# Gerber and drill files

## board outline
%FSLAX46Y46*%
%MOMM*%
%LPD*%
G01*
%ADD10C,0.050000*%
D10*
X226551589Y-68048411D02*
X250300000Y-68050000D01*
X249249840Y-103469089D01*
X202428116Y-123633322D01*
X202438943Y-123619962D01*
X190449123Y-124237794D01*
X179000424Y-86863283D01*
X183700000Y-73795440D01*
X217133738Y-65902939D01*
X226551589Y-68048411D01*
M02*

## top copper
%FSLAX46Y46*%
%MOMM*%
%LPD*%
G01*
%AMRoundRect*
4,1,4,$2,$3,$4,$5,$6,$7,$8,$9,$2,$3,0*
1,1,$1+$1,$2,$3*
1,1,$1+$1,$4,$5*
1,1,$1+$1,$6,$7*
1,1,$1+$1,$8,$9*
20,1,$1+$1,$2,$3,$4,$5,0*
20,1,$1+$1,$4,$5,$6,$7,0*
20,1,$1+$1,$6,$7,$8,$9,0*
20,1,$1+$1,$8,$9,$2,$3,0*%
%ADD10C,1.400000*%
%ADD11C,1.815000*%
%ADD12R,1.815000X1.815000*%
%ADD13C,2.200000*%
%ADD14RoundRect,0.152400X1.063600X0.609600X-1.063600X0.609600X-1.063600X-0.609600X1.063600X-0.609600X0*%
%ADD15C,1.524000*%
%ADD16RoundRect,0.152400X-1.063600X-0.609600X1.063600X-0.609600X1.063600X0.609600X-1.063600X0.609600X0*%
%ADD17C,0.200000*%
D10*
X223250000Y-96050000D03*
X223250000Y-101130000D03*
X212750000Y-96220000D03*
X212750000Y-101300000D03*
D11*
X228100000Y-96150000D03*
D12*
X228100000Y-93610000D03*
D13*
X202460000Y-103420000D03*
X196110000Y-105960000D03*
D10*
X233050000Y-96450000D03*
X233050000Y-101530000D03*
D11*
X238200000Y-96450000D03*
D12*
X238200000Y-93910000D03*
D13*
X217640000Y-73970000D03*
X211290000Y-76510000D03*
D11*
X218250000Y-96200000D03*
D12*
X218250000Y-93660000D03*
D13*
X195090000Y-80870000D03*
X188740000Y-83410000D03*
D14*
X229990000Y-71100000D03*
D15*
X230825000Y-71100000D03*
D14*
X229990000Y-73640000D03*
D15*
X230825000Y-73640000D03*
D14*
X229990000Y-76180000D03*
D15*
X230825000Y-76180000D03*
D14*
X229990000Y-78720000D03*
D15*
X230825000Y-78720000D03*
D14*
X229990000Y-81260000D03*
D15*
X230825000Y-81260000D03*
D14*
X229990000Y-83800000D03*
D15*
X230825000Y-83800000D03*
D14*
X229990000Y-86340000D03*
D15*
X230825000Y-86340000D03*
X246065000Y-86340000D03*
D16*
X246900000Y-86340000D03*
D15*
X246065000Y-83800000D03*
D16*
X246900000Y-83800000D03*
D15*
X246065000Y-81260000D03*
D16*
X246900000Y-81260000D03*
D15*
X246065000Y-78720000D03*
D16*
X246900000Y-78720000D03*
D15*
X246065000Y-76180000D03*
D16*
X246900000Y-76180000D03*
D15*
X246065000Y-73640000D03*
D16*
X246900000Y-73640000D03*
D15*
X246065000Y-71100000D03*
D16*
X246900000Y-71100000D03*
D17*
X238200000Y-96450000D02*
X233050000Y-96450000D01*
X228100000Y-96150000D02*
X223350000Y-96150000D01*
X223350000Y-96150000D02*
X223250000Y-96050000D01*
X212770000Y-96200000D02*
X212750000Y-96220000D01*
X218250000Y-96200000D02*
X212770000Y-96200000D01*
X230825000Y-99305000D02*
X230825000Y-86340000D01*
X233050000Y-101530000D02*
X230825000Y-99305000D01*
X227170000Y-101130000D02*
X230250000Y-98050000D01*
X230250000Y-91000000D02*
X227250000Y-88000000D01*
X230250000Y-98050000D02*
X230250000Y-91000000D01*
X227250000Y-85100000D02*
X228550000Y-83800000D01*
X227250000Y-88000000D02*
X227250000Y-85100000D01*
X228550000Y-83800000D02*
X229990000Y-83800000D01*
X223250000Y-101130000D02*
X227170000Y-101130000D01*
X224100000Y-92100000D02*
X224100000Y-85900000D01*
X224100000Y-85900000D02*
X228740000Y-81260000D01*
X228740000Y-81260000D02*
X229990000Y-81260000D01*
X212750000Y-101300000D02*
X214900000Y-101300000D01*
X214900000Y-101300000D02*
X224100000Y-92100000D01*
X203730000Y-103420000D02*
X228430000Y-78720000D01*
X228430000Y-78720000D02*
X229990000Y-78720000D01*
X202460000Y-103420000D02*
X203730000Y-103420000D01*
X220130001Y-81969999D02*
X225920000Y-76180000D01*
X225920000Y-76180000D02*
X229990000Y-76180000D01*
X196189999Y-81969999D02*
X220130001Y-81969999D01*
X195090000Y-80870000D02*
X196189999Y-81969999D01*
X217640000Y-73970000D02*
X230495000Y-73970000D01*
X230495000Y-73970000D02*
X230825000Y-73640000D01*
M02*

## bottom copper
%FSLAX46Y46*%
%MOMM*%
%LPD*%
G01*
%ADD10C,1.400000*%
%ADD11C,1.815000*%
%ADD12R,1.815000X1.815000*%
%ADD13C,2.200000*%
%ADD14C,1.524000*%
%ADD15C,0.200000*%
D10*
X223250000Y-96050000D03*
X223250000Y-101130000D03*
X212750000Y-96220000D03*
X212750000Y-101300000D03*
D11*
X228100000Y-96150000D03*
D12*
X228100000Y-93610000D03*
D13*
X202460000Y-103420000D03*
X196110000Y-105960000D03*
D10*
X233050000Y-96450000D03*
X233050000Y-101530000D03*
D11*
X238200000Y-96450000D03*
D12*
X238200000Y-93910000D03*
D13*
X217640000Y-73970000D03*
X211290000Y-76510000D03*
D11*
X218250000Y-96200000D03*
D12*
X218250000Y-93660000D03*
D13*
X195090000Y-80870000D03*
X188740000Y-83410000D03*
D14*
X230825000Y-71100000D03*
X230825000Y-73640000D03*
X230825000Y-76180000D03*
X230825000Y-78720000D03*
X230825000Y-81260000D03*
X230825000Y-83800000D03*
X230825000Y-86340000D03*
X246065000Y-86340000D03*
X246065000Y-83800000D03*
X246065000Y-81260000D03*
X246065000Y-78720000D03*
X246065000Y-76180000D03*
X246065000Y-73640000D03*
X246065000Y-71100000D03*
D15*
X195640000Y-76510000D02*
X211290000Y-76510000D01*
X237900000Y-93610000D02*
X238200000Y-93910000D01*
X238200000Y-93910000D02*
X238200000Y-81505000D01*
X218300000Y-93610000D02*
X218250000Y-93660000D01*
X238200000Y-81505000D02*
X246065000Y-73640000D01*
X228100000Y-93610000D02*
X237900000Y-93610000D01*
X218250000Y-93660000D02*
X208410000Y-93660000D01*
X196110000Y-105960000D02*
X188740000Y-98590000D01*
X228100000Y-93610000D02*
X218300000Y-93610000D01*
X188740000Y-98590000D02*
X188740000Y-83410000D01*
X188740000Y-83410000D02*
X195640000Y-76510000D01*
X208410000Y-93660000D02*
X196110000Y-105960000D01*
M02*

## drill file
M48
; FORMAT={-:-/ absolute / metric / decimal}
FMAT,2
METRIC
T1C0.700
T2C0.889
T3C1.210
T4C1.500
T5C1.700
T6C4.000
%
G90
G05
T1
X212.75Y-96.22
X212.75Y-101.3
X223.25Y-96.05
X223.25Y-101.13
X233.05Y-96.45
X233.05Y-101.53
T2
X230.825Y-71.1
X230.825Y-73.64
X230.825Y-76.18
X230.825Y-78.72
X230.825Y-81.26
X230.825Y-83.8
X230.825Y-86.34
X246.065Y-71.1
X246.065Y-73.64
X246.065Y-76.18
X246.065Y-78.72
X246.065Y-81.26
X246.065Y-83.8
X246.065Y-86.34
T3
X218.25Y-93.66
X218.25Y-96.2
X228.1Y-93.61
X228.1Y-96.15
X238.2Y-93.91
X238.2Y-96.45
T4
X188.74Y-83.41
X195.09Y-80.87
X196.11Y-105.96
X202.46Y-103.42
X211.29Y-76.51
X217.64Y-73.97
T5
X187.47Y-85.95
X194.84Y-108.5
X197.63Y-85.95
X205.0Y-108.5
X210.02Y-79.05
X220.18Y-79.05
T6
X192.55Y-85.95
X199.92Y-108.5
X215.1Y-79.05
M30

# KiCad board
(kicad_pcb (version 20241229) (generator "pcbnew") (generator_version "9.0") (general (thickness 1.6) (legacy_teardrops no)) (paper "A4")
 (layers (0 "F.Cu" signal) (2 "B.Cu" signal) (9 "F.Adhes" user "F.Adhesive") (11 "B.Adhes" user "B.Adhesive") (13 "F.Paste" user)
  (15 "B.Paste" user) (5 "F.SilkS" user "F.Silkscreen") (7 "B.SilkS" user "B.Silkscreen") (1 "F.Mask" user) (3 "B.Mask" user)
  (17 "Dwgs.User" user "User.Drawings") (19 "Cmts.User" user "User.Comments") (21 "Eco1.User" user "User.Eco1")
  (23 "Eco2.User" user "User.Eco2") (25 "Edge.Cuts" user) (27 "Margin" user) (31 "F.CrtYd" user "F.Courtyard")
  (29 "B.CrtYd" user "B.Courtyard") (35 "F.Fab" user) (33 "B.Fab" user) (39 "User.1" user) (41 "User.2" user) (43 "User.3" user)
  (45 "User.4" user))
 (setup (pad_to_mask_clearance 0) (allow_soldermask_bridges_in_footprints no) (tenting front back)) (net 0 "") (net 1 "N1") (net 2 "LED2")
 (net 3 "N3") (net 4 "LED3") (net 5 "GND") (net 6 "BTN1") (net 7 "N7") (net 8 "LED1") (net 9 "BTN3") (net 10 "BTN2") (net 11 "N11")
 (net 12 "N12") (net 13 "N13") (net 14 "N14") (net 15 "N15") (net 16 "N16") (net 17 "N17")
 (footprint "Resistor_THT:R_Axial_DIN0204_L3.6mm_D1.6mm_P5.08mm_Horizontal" (layer "F.Cu") (at 223.25 96.05 -90)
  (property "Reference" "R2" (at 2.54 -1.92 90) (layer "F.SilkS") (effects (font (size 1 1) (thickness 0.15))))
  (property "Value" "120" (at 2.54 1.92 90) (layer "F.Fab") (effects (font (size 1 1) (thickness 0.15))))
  (pad "1" thru_hole circle (at 0 0 270) (size 1.4 1.4) (drill 0.7) (layers "*.Cu" "*.Mask") (remove_unused_layers no) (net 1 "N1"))
  (pad "2" thru_hole circle (at 5.08 0 270) (size 1.4 1.4) (drill 0.7) (layers "*.Cu" "*.Mask") (remove_unused_layers no) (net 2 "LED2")))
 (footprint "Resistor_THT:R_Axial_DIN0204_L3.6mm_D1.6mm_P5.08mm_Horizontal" (layer "F.Cu") (at 212.75 96.22 -90)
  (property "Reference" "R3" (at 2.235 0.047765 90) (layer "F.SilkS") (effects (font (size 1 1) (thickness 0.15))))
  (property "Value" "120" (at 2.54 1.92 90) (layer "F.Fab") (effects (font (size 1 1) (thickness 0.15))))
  (pad "1" thru_hole circle (at 0 0 270) (size 1.4 1.4) (drill 0.7) (layers "*.Cu" "*.Mask") (remove_unused_layers no) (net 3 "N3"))
  (pad "2" thru_hole circle (at 5.08 0 270) (size 1.4 1.4) (drill 0.7) (layers "*.Cu" "*.Mask") (remove_unused_layers no) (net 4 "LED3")))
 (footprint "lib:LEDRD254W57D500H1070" (layer "F.Cu") (at 228.1 94.88 -90)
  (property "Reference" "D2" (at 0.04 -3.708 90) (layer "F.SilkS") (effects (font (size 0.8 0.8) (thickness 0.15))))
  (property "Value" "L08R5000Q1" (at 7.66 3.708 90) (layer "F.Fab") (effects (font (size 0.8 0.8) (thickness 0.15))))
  (pad "A" thru_hole circle (at 1.27 0 270) (size 1.815 1.815) (drill 1.21) (layers "*.Cu" "*.Mask") (remove_unused_layers no) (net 1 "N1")
   (solder_mask_margin 0.102))
  (pad "C" thru_hole rect (at -1.27 0 270) (size 1.815 1.815) (drill 1.21) (layers "*.Cu" "*.Mask") (remove_unused_layers no) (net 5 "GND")
   (solder_mask_margin 0.102)))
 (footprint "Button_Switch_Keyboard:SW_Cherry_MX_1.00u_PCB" (layer "F.Cu") (at 202.46 103.42)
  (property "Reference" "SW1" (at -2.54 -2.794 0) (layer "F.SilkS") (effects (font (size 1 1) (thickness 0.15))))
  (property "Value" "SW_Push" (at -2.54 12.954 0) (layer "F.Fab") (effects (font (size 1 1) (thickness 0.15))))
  (pad "" np_thru_hole circle (at -7.62 5.08) (size 1.7 1.7) (drill 1.7) (layers "*.Cu" "*.Mask"))
  (pad "" np_thru_hole circle (at -2.54 5.08) (size 4 4) (drill 4) (layers "*.Cu" "*.Mask"))
  (pad "" np_thru_hole circle (at 2.54 5.08) (size 1.7 1.7) (drill 1.7) (layers "*.Cu" "*.Mask"))
  (pad "1" thru_hole circle (at 0 0) (size 2.2 2.2) (drill 1.5) (layers "*.Cu" "*.Mask") (remove_unused_layers no) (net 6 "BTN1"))
  (pad "2" thru_hole circle (at -6.35 2.54) (size 2.2 2.2) (drill 1.5) (layers "*.Cu" "*.Mask") (remove_unused_layers no) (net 5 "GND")))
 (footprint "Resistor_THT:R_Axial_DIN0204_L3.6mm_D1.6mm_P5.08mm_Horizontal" (layer "F.Cu") (at 233.05 96.45 -90)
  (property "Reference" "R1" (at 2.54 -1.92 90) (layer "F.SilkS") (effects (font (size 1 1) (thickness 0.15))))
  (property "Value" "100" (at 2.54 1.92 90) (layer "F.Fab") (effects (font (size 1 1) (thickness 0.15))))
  (pad "1" thru_hole circle (at 0 0 270) (size 1.4 1.4) (drill 0.7) (layers "*.Cu" "*.Mask") (remove_unused_layers no) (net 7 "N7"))
  (pad "2" thru_hole circle (at 5.08 0 270) (size 1.4 1.4) (drill 0.7) (layers "*.Cu" "*.Mask") (remove_unused_layers no) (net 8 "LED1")))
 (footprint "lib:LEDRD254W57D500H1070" (layer "F.Cu") (at 238.2 95.18 -90)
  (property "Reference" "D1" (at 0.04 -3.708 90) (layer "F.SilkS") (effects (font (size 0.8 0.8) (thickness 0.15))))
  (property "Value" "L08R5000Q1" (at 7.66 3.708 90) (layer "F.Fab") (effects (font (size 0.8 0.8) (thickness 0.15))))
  (pad "A" thru_hole circle (at 1.27 0 270) (size 1.815 1.815) (drill 1.21) (layers "*.Cu" "*.Mask") (remove_unused_layers no) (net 7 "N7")
   (solder_mask_margin 0.102))
  (pad "C" thru_hole rect (at -1.27 0 270) (size 1.815 1.815) (drill 1.21) (layers "*.Cu" "*.Mask") (remove_unused_layers no) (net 5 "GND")
   (solder_mask_margin 0.102)))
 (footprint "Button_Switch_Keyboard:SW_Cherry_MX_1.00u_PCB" (layer "F.Cu") (at 217.64 73.97)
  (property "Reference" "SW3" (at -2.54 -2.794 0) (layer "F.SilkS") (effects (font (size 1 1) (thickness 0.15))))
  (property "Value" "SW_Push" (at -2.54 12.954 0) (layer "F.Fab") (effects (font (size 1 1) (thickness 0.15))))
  (pad "" np_thru_hole circle (at -7.62 5.08) (size 1.7 1.7) (drill 1.7) (layers "*.Cu" "*.Mask"))
  (pad "" np_thru_hole circle (at -2.54 5.08) (size 4 4) (drill 4) (layers "*.Cu" "*.Mask"))
  (pad "" np_thru_hole circle (at 2.54 5.08) (size 1.7 1.7) (drill 1.7) (layers "*.Cu" "*.Mask"))
  (pad "1" thru_hole circle (at 0 0) (size 2.2 2.2) (drill 1.5) (layers "*.Cu" "*.Mask") (remove_unused_layers no) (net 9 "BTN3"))
  (pad "2" thru_hole circle (at -6.35 2.54) (size 2.2 2.2) (drill 1.5) (layers "*.Cu" "*.Mask") (remove_unused_layers no) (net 5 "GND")))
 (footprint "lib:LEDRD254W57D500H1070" (layer "F.Cu") (at 218.25 94.93 -90)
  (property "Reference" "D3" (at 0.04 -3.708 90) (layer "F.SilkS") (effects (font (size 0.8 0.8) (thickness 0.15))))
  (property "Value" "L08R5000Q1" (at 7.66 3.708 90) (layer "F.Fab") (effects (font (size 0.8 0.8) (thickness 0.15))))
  (pad "A" thru_hole circle (at 1.27 0 270) (size 1.815 1.815) (drill 1.21) (layers "*.Cu" "*.Mask") (remove_unused_layers no) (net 3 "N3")
   (solder_mask_margin 0.102))
  (pad "C" thru_hole rect (at -1.27 0 270) (size 1.815 1.815) (drill 1.21) (layers "*.Cu" "*.Mask") (remove_unused_layers no) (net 5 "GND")
   (solder_mask_margin 0.102)))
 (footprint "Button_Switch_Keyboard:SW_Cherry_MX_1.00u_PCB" (layer "F.Cu") (at 195.09 80.87)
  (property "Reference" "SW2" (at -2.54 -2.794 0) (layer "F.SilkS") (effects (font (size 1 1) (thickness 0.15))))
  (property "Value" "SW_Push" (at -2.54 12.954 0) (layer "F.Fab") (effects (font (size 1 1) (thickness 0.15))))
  (pad "" np_thru_hole circle (at -7.62 5.08) (size 1.7 1.7) (drill 1.7) (layers "*.Cu" "*.Mask"))
  (pad "" np_thru_hole circle (at -2.54 5.08) (size 4 4) (drill 4) (layers "*.Cu" "*.Mask"))
  (pad "" np_thru_hole circle (at 2.54 5.08) (size 1.7 1.7) (drill 1.7) (layers "*.Cu" "*.Mask"))
  (pad "1" thru_hole circle (at 0 0) (size 2.2 2.2) (drill 1.5) (layers "*.Cu" "*.Mask") (remove_unused_layers no) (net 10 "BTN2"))
  (pad "2" thru_hole circle (at -6.35 2.54) (size 2.2 2.2) (drill 1.5) (layers "*.Cu" "*.Mask") (remove_unused_layers no) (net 5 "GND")))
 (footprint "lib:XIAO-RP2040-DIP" (layer "F.Cu") (at 238.445 78.72)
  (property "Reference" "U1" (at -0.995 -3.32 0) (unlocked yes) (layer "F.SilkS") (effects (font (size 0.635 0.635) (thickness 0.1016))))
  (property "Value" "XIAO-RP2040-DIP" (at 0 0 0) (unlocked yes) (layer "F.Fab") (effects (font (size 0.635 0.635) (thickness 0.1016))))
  (pad "1" smd roundrect (at -8.455 -7.62 180) (size 2.432 1.524) (layers "F.Cu" "F.Mask") (roundrect_rratio 0.1) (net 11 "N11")
   (thermal_bridge_angle 45))
  (pad "1" thru_hole circle (at -7.62 -7.62 180) (size 1.524 1.524) (drill 0.889) (layers "*.Cu" "*.Mask") (remove_unused_layers no)
   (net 11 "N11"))
  (pad "2" smd roundrect (at -8.455 -5.08 180) (size 2.432 1.524) (layers "F.Cu" "F.Mask") (roundrect_rratio 0.1) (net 9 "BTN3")
   (thermal_bridge_angle 45))
  (pad "2" thru_hole circle (at -7.62 -5.08 180) (size 1.524 1.524) (drill 0.889) (layers "*.Cu" "*.Mask") (remove_unused_layers no)
   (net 9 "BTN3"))
  (pad "3" smd roundrect (at -8.455 -2.54 180) (size 2.432 1.524) (layers "F.Cu" "F.Mask") (roundrect_rratio 0.1) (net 10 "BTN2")
   (thermal_bridge_angle 45))
  (pad "3" thru_hole circle (at -7.62 -2.54 180) (size 1.524 1.524) (drill 0.889) (layers "*.Cu" "*.Mask") (remove_unused_layers no)
   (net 10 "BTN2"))
  (pad "4" smd roundrect (at -8.455 0 180) (size 2.432 1.524) (layers "F.Cu" "F.Mask") (roundrect_rratio 0.1) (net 6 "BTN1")
   (thermal_bridge_angle 45))
  (pad "4" thru_hole circle (at -7.62 0 180) (size 1.524 1.524) (drill 0.889) (layers "*.Cu" "*.Mask") (remove_unused_layers no)
   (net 6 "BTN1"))
  (pad "5" smd roundrect (at -8.455 2.54 180) (size 2.432 1.524) (layers "F.Cu" "F.Mask") (roundrect_rratio 0.1) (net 4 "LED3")
   (thermal_bridge_angle 45))
  (pad "5" thru_hole circle (at -7.62 2.54 180) (size 1.524 1.524) (drill 0.889) (layers "*.Cu" "*.Mask") (remove_unused_layers no)
   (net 4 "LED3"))
  (pad "6" smd roundrect (at -8.455 5.08 180) (size 2.432 1.524) (layers "F.Cu" "F.Mask") (roundrect_rratio 0.1) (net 2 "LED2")
   (thermal_bridge_angle 45))
  (pad "6" thru_hole circle (at -7.62 5.08 180) (size 1.524 1.524) (drill 0.889) (layers "*.Cu" "*.Mask") (remove_unused_layers no)
   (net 2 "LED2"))
  (pad "7" smd roundrect (at -8.455 7.62 180) (size 2.432 1.524) (layers "F.Cu" "F.Mask") (roundrect_rratio 0.1) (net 8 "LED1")
   (thermal_bridge_angle 45))
  (pad "7" thru_hole circle (at -7.62 7.62 180) (size 1.524 1.524) (drill 0.889) (layers "*.Cu" "*.Mask") (remove_unused_layers no)
   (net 8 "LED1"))
  (pad "8" thru_hole circle (at 7.62 7.62) (size 1.524 1.524) (drill 0.889) (layers "*.Cu" "*.Mask") (remove_unused_layers no)
   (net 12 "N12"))
  (pad "8" smd roundrect (at 8.455 7.62) (size 2.432 1.524) (layers "F.Cu" "F.Mask") (roundrect_rratio 0.1) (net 12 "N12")
   (thermal_bridge_angle 45))
  (pad "9" thru_hole circle (at 7.62 5.08) (size 1.524 1.524) (drill 0.889) (layers "*.Cu" "*.Mask") (remove_unused_layers no)
   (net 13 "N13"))
  (pad "9" smd roundrect (at 8.455 5.08) (size 2.432 1.524) (layers "F.Cu" "F.Mask") (roundrect_rratio 0.1) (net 13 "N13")
   (thermal_bridge_angle 45))
  (pad "10" thru_hole circle (at 7.62 2.54) (size 1.524 1.524) (drill 0.889) (layers "*.Cu" "*.Mask") (remove_unused_layers no)
   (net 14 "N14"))
  (pad "10" smd roundrect (at 8.455 2.54) (size 2.432 1.524) (layers "F.Cu" "F.Mask") (roundrect_rratio 0.1) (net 14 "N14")
   (thermal_bridge_angle 45))
  (pad "11" thru_hole circle (at 7.62 0) (size 1.524 1.524) (drill 0.889) (layers "*.Cu" "*.Mask") (remove_unused_layers no) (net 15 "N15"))
  (pad "11" smd roundrect (at 8.455 0) (size 2.432 1.524) (layers "F.Cu" "F.Mask") (roundrect_rratio 0.1) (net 15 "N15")
   (thermal_bridge_angle 45))
  (pad "12" thru_hole circle (at 7.62 -2.54) (size 1.524 1.524) (drill 0.889) (layers "*.Cu" "*.Mask") (remove_unused_layers no)
   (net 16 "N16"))
  (pad "12" smd roundrect (at 8.455 -2.54) (size 2.432 1.524) (layers "F.Cu" "F.Mask") (roundrect_rratio 0.1) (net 16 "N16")
   (thermal_bridge_angle 45))
  (pad "13" thru_hole circle (at 7.62 -5.08) (size 1.524 1.524) (drill 0.889) (layers "*.Cu" "*.Mask") (remove_unused_layers no)
   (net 5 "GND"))
  (pad "13" smd roundrect (at 8.455 -5.08) (size 2.432 1.524) (layers "F.Cu" "F.Mask") (roundrect_rratio 0.1) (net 5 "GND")
   (thermal_bridge_angle 45))
  (pad "14" thru_hole circle (at 7.62 -7.62) (size 1.524 1.524) (drill 0.889) (layers "*.Cu" "*.Mask") (remove_unused_layers no)
   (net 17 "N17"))
  (pad "14" smd roundrect (at 8.455 -7.62) (size 2.432 1.524) (layers "F.Cu" "F.Mask") (roundrect_rratio 0.1) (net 17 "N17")
   (thermal_bridge_angle 45)))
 (gr_poly
  (pts (xy 226.551589 68.048411) (xy 250.3 68.05) (xy 249.24984 103.469089) (xy 202.428116 123.633322) (xy 202.438943 123.619962)
   (xy 190.449123 124.237794) (xy 179.000424 86.863283) (xy 183.7 73.79544) (xy 217.133738 65.902939))
  (stroke (width 0.05) (type solid)) (fill no) (layer "Edge.Cuts"))
 (segment (start 238.2 96.45) (end 233.05 96.45) (width 0.2) (layer "F.Cu") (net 7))
 (segment (start 195.64 76.51) (end 211.29 76.51) (width 0.2) (layer "B.Cu") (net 5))
 (segment (start 237.9 93.61) (end 238.2 93.91) (width 0.2) (layer "B.Cu") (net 5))
 (segment (start 238.2 93.91) (end 238.2 81.505) (width 0.2) (layer "B.Cu") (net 5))
 (segment (start 218.3 93.61) (end 218.25 93.66) (width 0.2) (layer "B.Cu") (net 5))
 (segment (start 238.2 81.505) (end 246.065 73.64) (width 0.2) (layer "B.Cu") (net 5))
 (segment (start 228.1 93.61) (end 237.9 93.61) (width 0.2) (layer "B.Cu") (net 5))
 (segment (start 218.25 93.66) (end 208.41 93.66) (width 0.2) (layer "B.Cu") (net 5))
 (segment (start 196.11 105.96) (end 188.74 98.59) (width 0.2) (layer "B.Cu") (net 5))
 (segment (start 228.1 93.61) (end 218.3 93.61) (width 0.2) (layer "B.Cu") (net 5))
 (segment (start 188.74 98.59) (end 188.74 83.41) (width 0.2) (layer "B.Cu") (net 5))
 (segment (start 188.74 83.41) (end 195.64 76.51) (width 0.2) (layer "B.Cu") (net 5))
 (segment (start 208.41 93.66) (end 196.11 105.96) (width 0.2) (layer "B.Cu") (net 5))
 (segment (start 228.1 96.15) (end 223.35 96.15) (width 0.2) (layer "F.Cu") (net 1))
 (segment (start 223.35 96.15) (end 223.25 96.05) (width 0.2) (layer "F.Cu") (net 1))
 (segment (start 212.77 96.2) (end 212.75 96.22) (width 0.2) (layer "F.Cu") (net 3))
 (segment (start 218.25 96.2) (end 212.77 96.2) (width 0.2) (layer "F.Cu") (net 3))
 (segment (start 230.825 99.305) (end 230.825 86.34) (width 0.2) (layer "F.Cu") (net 8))
 (segment (start 233.05 101.53) (end 230.825 99.305) (width 0.2) (layer "F.Cu") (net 8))
 (segment (start 227.17 101.13) (end 230.25 98.05) (width 0.2) (layer "F.Cu") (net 2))
 (segment (start 230.25 91) (end 227.25 88) (width 0.2) (layer "F.Cu") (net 2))
 (segment (start 230.25 98.05) (end 230.25 91) (width 0.2) (layer "F.Cu") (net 2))
 (segment (start 227.25 85.1) (end 228.55 83.8) (width 0.2) (layer "F.Cu") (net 2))
 (segment (start 227.25 88) (end 227.25 85.1) (width 0.2) (layer "F.Cu") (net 2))
 (segment (start 228.55 83.8) (end 229.99 83.8) (width 0.2) (layer "F.Cu") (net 2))
 (segment (start 223.25 101.13) (end 227.17 101.13) (width 0.2) (layer "F.Cu") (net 2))
 (segment (start 224.1 92.1) (end 224.1 85.9) (width 0.2) (layer "F.Cu") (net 4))
 (segment (start 224.1 85.9) (end 228.74 81.26) (width 0.2) (layer "F.Cu") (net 4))
 (segment (start 228.74 81.26) (end 229.99 81.26) (width 0.2) (layer "F.Cu") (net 4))
 (segment (start 212.75 101.3) (end 214.9 101.3) (width 0.2) (layer "F.Cu") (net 4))
 (segment (start 214.9 101.3) (end 224.1 92.1) (width 0.2) (layer "F.Cu") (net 4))
 (segment (start 203.73 103.42) (end 228.43 78.72) (width 0.2) (layer "F.Cu") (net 6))
 (segment (start 228.43 78.72) (end 229.99 78.72) (width 0.2) (layer "F.Cu") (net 6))
 (segment (start 202.46 103.42) (end 203.73 103.42) (width 0.2) (layer "F.Cu") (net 6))
 (segment (start 220.130001 81.969999) (end 225.92 76.18) (width 0.2) (layer "F.Cu") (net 10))
 (segment (start 225.92 76.18) (end 229.99 76.18) (width 0.2) (layer "F.Cu") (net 10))
 (segment (start 196.189999 81.969999) (end 220.130001 81.969999) (width 0.2) (layer "F.Cu") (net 10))
 (segment (start 195.09 80.87) (end 196.189999 81.969999) (width 0.2) (layer "F.Cu") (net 10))
 (segment (start 217.64 73.97) (end 230.495 73.97) (width 0.2) (layer "F.Cu") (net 9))
 (segment (start 230.495 73.97) (end 230.825 73.64) (width 0.2) (layer "F.Cu") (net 9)))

